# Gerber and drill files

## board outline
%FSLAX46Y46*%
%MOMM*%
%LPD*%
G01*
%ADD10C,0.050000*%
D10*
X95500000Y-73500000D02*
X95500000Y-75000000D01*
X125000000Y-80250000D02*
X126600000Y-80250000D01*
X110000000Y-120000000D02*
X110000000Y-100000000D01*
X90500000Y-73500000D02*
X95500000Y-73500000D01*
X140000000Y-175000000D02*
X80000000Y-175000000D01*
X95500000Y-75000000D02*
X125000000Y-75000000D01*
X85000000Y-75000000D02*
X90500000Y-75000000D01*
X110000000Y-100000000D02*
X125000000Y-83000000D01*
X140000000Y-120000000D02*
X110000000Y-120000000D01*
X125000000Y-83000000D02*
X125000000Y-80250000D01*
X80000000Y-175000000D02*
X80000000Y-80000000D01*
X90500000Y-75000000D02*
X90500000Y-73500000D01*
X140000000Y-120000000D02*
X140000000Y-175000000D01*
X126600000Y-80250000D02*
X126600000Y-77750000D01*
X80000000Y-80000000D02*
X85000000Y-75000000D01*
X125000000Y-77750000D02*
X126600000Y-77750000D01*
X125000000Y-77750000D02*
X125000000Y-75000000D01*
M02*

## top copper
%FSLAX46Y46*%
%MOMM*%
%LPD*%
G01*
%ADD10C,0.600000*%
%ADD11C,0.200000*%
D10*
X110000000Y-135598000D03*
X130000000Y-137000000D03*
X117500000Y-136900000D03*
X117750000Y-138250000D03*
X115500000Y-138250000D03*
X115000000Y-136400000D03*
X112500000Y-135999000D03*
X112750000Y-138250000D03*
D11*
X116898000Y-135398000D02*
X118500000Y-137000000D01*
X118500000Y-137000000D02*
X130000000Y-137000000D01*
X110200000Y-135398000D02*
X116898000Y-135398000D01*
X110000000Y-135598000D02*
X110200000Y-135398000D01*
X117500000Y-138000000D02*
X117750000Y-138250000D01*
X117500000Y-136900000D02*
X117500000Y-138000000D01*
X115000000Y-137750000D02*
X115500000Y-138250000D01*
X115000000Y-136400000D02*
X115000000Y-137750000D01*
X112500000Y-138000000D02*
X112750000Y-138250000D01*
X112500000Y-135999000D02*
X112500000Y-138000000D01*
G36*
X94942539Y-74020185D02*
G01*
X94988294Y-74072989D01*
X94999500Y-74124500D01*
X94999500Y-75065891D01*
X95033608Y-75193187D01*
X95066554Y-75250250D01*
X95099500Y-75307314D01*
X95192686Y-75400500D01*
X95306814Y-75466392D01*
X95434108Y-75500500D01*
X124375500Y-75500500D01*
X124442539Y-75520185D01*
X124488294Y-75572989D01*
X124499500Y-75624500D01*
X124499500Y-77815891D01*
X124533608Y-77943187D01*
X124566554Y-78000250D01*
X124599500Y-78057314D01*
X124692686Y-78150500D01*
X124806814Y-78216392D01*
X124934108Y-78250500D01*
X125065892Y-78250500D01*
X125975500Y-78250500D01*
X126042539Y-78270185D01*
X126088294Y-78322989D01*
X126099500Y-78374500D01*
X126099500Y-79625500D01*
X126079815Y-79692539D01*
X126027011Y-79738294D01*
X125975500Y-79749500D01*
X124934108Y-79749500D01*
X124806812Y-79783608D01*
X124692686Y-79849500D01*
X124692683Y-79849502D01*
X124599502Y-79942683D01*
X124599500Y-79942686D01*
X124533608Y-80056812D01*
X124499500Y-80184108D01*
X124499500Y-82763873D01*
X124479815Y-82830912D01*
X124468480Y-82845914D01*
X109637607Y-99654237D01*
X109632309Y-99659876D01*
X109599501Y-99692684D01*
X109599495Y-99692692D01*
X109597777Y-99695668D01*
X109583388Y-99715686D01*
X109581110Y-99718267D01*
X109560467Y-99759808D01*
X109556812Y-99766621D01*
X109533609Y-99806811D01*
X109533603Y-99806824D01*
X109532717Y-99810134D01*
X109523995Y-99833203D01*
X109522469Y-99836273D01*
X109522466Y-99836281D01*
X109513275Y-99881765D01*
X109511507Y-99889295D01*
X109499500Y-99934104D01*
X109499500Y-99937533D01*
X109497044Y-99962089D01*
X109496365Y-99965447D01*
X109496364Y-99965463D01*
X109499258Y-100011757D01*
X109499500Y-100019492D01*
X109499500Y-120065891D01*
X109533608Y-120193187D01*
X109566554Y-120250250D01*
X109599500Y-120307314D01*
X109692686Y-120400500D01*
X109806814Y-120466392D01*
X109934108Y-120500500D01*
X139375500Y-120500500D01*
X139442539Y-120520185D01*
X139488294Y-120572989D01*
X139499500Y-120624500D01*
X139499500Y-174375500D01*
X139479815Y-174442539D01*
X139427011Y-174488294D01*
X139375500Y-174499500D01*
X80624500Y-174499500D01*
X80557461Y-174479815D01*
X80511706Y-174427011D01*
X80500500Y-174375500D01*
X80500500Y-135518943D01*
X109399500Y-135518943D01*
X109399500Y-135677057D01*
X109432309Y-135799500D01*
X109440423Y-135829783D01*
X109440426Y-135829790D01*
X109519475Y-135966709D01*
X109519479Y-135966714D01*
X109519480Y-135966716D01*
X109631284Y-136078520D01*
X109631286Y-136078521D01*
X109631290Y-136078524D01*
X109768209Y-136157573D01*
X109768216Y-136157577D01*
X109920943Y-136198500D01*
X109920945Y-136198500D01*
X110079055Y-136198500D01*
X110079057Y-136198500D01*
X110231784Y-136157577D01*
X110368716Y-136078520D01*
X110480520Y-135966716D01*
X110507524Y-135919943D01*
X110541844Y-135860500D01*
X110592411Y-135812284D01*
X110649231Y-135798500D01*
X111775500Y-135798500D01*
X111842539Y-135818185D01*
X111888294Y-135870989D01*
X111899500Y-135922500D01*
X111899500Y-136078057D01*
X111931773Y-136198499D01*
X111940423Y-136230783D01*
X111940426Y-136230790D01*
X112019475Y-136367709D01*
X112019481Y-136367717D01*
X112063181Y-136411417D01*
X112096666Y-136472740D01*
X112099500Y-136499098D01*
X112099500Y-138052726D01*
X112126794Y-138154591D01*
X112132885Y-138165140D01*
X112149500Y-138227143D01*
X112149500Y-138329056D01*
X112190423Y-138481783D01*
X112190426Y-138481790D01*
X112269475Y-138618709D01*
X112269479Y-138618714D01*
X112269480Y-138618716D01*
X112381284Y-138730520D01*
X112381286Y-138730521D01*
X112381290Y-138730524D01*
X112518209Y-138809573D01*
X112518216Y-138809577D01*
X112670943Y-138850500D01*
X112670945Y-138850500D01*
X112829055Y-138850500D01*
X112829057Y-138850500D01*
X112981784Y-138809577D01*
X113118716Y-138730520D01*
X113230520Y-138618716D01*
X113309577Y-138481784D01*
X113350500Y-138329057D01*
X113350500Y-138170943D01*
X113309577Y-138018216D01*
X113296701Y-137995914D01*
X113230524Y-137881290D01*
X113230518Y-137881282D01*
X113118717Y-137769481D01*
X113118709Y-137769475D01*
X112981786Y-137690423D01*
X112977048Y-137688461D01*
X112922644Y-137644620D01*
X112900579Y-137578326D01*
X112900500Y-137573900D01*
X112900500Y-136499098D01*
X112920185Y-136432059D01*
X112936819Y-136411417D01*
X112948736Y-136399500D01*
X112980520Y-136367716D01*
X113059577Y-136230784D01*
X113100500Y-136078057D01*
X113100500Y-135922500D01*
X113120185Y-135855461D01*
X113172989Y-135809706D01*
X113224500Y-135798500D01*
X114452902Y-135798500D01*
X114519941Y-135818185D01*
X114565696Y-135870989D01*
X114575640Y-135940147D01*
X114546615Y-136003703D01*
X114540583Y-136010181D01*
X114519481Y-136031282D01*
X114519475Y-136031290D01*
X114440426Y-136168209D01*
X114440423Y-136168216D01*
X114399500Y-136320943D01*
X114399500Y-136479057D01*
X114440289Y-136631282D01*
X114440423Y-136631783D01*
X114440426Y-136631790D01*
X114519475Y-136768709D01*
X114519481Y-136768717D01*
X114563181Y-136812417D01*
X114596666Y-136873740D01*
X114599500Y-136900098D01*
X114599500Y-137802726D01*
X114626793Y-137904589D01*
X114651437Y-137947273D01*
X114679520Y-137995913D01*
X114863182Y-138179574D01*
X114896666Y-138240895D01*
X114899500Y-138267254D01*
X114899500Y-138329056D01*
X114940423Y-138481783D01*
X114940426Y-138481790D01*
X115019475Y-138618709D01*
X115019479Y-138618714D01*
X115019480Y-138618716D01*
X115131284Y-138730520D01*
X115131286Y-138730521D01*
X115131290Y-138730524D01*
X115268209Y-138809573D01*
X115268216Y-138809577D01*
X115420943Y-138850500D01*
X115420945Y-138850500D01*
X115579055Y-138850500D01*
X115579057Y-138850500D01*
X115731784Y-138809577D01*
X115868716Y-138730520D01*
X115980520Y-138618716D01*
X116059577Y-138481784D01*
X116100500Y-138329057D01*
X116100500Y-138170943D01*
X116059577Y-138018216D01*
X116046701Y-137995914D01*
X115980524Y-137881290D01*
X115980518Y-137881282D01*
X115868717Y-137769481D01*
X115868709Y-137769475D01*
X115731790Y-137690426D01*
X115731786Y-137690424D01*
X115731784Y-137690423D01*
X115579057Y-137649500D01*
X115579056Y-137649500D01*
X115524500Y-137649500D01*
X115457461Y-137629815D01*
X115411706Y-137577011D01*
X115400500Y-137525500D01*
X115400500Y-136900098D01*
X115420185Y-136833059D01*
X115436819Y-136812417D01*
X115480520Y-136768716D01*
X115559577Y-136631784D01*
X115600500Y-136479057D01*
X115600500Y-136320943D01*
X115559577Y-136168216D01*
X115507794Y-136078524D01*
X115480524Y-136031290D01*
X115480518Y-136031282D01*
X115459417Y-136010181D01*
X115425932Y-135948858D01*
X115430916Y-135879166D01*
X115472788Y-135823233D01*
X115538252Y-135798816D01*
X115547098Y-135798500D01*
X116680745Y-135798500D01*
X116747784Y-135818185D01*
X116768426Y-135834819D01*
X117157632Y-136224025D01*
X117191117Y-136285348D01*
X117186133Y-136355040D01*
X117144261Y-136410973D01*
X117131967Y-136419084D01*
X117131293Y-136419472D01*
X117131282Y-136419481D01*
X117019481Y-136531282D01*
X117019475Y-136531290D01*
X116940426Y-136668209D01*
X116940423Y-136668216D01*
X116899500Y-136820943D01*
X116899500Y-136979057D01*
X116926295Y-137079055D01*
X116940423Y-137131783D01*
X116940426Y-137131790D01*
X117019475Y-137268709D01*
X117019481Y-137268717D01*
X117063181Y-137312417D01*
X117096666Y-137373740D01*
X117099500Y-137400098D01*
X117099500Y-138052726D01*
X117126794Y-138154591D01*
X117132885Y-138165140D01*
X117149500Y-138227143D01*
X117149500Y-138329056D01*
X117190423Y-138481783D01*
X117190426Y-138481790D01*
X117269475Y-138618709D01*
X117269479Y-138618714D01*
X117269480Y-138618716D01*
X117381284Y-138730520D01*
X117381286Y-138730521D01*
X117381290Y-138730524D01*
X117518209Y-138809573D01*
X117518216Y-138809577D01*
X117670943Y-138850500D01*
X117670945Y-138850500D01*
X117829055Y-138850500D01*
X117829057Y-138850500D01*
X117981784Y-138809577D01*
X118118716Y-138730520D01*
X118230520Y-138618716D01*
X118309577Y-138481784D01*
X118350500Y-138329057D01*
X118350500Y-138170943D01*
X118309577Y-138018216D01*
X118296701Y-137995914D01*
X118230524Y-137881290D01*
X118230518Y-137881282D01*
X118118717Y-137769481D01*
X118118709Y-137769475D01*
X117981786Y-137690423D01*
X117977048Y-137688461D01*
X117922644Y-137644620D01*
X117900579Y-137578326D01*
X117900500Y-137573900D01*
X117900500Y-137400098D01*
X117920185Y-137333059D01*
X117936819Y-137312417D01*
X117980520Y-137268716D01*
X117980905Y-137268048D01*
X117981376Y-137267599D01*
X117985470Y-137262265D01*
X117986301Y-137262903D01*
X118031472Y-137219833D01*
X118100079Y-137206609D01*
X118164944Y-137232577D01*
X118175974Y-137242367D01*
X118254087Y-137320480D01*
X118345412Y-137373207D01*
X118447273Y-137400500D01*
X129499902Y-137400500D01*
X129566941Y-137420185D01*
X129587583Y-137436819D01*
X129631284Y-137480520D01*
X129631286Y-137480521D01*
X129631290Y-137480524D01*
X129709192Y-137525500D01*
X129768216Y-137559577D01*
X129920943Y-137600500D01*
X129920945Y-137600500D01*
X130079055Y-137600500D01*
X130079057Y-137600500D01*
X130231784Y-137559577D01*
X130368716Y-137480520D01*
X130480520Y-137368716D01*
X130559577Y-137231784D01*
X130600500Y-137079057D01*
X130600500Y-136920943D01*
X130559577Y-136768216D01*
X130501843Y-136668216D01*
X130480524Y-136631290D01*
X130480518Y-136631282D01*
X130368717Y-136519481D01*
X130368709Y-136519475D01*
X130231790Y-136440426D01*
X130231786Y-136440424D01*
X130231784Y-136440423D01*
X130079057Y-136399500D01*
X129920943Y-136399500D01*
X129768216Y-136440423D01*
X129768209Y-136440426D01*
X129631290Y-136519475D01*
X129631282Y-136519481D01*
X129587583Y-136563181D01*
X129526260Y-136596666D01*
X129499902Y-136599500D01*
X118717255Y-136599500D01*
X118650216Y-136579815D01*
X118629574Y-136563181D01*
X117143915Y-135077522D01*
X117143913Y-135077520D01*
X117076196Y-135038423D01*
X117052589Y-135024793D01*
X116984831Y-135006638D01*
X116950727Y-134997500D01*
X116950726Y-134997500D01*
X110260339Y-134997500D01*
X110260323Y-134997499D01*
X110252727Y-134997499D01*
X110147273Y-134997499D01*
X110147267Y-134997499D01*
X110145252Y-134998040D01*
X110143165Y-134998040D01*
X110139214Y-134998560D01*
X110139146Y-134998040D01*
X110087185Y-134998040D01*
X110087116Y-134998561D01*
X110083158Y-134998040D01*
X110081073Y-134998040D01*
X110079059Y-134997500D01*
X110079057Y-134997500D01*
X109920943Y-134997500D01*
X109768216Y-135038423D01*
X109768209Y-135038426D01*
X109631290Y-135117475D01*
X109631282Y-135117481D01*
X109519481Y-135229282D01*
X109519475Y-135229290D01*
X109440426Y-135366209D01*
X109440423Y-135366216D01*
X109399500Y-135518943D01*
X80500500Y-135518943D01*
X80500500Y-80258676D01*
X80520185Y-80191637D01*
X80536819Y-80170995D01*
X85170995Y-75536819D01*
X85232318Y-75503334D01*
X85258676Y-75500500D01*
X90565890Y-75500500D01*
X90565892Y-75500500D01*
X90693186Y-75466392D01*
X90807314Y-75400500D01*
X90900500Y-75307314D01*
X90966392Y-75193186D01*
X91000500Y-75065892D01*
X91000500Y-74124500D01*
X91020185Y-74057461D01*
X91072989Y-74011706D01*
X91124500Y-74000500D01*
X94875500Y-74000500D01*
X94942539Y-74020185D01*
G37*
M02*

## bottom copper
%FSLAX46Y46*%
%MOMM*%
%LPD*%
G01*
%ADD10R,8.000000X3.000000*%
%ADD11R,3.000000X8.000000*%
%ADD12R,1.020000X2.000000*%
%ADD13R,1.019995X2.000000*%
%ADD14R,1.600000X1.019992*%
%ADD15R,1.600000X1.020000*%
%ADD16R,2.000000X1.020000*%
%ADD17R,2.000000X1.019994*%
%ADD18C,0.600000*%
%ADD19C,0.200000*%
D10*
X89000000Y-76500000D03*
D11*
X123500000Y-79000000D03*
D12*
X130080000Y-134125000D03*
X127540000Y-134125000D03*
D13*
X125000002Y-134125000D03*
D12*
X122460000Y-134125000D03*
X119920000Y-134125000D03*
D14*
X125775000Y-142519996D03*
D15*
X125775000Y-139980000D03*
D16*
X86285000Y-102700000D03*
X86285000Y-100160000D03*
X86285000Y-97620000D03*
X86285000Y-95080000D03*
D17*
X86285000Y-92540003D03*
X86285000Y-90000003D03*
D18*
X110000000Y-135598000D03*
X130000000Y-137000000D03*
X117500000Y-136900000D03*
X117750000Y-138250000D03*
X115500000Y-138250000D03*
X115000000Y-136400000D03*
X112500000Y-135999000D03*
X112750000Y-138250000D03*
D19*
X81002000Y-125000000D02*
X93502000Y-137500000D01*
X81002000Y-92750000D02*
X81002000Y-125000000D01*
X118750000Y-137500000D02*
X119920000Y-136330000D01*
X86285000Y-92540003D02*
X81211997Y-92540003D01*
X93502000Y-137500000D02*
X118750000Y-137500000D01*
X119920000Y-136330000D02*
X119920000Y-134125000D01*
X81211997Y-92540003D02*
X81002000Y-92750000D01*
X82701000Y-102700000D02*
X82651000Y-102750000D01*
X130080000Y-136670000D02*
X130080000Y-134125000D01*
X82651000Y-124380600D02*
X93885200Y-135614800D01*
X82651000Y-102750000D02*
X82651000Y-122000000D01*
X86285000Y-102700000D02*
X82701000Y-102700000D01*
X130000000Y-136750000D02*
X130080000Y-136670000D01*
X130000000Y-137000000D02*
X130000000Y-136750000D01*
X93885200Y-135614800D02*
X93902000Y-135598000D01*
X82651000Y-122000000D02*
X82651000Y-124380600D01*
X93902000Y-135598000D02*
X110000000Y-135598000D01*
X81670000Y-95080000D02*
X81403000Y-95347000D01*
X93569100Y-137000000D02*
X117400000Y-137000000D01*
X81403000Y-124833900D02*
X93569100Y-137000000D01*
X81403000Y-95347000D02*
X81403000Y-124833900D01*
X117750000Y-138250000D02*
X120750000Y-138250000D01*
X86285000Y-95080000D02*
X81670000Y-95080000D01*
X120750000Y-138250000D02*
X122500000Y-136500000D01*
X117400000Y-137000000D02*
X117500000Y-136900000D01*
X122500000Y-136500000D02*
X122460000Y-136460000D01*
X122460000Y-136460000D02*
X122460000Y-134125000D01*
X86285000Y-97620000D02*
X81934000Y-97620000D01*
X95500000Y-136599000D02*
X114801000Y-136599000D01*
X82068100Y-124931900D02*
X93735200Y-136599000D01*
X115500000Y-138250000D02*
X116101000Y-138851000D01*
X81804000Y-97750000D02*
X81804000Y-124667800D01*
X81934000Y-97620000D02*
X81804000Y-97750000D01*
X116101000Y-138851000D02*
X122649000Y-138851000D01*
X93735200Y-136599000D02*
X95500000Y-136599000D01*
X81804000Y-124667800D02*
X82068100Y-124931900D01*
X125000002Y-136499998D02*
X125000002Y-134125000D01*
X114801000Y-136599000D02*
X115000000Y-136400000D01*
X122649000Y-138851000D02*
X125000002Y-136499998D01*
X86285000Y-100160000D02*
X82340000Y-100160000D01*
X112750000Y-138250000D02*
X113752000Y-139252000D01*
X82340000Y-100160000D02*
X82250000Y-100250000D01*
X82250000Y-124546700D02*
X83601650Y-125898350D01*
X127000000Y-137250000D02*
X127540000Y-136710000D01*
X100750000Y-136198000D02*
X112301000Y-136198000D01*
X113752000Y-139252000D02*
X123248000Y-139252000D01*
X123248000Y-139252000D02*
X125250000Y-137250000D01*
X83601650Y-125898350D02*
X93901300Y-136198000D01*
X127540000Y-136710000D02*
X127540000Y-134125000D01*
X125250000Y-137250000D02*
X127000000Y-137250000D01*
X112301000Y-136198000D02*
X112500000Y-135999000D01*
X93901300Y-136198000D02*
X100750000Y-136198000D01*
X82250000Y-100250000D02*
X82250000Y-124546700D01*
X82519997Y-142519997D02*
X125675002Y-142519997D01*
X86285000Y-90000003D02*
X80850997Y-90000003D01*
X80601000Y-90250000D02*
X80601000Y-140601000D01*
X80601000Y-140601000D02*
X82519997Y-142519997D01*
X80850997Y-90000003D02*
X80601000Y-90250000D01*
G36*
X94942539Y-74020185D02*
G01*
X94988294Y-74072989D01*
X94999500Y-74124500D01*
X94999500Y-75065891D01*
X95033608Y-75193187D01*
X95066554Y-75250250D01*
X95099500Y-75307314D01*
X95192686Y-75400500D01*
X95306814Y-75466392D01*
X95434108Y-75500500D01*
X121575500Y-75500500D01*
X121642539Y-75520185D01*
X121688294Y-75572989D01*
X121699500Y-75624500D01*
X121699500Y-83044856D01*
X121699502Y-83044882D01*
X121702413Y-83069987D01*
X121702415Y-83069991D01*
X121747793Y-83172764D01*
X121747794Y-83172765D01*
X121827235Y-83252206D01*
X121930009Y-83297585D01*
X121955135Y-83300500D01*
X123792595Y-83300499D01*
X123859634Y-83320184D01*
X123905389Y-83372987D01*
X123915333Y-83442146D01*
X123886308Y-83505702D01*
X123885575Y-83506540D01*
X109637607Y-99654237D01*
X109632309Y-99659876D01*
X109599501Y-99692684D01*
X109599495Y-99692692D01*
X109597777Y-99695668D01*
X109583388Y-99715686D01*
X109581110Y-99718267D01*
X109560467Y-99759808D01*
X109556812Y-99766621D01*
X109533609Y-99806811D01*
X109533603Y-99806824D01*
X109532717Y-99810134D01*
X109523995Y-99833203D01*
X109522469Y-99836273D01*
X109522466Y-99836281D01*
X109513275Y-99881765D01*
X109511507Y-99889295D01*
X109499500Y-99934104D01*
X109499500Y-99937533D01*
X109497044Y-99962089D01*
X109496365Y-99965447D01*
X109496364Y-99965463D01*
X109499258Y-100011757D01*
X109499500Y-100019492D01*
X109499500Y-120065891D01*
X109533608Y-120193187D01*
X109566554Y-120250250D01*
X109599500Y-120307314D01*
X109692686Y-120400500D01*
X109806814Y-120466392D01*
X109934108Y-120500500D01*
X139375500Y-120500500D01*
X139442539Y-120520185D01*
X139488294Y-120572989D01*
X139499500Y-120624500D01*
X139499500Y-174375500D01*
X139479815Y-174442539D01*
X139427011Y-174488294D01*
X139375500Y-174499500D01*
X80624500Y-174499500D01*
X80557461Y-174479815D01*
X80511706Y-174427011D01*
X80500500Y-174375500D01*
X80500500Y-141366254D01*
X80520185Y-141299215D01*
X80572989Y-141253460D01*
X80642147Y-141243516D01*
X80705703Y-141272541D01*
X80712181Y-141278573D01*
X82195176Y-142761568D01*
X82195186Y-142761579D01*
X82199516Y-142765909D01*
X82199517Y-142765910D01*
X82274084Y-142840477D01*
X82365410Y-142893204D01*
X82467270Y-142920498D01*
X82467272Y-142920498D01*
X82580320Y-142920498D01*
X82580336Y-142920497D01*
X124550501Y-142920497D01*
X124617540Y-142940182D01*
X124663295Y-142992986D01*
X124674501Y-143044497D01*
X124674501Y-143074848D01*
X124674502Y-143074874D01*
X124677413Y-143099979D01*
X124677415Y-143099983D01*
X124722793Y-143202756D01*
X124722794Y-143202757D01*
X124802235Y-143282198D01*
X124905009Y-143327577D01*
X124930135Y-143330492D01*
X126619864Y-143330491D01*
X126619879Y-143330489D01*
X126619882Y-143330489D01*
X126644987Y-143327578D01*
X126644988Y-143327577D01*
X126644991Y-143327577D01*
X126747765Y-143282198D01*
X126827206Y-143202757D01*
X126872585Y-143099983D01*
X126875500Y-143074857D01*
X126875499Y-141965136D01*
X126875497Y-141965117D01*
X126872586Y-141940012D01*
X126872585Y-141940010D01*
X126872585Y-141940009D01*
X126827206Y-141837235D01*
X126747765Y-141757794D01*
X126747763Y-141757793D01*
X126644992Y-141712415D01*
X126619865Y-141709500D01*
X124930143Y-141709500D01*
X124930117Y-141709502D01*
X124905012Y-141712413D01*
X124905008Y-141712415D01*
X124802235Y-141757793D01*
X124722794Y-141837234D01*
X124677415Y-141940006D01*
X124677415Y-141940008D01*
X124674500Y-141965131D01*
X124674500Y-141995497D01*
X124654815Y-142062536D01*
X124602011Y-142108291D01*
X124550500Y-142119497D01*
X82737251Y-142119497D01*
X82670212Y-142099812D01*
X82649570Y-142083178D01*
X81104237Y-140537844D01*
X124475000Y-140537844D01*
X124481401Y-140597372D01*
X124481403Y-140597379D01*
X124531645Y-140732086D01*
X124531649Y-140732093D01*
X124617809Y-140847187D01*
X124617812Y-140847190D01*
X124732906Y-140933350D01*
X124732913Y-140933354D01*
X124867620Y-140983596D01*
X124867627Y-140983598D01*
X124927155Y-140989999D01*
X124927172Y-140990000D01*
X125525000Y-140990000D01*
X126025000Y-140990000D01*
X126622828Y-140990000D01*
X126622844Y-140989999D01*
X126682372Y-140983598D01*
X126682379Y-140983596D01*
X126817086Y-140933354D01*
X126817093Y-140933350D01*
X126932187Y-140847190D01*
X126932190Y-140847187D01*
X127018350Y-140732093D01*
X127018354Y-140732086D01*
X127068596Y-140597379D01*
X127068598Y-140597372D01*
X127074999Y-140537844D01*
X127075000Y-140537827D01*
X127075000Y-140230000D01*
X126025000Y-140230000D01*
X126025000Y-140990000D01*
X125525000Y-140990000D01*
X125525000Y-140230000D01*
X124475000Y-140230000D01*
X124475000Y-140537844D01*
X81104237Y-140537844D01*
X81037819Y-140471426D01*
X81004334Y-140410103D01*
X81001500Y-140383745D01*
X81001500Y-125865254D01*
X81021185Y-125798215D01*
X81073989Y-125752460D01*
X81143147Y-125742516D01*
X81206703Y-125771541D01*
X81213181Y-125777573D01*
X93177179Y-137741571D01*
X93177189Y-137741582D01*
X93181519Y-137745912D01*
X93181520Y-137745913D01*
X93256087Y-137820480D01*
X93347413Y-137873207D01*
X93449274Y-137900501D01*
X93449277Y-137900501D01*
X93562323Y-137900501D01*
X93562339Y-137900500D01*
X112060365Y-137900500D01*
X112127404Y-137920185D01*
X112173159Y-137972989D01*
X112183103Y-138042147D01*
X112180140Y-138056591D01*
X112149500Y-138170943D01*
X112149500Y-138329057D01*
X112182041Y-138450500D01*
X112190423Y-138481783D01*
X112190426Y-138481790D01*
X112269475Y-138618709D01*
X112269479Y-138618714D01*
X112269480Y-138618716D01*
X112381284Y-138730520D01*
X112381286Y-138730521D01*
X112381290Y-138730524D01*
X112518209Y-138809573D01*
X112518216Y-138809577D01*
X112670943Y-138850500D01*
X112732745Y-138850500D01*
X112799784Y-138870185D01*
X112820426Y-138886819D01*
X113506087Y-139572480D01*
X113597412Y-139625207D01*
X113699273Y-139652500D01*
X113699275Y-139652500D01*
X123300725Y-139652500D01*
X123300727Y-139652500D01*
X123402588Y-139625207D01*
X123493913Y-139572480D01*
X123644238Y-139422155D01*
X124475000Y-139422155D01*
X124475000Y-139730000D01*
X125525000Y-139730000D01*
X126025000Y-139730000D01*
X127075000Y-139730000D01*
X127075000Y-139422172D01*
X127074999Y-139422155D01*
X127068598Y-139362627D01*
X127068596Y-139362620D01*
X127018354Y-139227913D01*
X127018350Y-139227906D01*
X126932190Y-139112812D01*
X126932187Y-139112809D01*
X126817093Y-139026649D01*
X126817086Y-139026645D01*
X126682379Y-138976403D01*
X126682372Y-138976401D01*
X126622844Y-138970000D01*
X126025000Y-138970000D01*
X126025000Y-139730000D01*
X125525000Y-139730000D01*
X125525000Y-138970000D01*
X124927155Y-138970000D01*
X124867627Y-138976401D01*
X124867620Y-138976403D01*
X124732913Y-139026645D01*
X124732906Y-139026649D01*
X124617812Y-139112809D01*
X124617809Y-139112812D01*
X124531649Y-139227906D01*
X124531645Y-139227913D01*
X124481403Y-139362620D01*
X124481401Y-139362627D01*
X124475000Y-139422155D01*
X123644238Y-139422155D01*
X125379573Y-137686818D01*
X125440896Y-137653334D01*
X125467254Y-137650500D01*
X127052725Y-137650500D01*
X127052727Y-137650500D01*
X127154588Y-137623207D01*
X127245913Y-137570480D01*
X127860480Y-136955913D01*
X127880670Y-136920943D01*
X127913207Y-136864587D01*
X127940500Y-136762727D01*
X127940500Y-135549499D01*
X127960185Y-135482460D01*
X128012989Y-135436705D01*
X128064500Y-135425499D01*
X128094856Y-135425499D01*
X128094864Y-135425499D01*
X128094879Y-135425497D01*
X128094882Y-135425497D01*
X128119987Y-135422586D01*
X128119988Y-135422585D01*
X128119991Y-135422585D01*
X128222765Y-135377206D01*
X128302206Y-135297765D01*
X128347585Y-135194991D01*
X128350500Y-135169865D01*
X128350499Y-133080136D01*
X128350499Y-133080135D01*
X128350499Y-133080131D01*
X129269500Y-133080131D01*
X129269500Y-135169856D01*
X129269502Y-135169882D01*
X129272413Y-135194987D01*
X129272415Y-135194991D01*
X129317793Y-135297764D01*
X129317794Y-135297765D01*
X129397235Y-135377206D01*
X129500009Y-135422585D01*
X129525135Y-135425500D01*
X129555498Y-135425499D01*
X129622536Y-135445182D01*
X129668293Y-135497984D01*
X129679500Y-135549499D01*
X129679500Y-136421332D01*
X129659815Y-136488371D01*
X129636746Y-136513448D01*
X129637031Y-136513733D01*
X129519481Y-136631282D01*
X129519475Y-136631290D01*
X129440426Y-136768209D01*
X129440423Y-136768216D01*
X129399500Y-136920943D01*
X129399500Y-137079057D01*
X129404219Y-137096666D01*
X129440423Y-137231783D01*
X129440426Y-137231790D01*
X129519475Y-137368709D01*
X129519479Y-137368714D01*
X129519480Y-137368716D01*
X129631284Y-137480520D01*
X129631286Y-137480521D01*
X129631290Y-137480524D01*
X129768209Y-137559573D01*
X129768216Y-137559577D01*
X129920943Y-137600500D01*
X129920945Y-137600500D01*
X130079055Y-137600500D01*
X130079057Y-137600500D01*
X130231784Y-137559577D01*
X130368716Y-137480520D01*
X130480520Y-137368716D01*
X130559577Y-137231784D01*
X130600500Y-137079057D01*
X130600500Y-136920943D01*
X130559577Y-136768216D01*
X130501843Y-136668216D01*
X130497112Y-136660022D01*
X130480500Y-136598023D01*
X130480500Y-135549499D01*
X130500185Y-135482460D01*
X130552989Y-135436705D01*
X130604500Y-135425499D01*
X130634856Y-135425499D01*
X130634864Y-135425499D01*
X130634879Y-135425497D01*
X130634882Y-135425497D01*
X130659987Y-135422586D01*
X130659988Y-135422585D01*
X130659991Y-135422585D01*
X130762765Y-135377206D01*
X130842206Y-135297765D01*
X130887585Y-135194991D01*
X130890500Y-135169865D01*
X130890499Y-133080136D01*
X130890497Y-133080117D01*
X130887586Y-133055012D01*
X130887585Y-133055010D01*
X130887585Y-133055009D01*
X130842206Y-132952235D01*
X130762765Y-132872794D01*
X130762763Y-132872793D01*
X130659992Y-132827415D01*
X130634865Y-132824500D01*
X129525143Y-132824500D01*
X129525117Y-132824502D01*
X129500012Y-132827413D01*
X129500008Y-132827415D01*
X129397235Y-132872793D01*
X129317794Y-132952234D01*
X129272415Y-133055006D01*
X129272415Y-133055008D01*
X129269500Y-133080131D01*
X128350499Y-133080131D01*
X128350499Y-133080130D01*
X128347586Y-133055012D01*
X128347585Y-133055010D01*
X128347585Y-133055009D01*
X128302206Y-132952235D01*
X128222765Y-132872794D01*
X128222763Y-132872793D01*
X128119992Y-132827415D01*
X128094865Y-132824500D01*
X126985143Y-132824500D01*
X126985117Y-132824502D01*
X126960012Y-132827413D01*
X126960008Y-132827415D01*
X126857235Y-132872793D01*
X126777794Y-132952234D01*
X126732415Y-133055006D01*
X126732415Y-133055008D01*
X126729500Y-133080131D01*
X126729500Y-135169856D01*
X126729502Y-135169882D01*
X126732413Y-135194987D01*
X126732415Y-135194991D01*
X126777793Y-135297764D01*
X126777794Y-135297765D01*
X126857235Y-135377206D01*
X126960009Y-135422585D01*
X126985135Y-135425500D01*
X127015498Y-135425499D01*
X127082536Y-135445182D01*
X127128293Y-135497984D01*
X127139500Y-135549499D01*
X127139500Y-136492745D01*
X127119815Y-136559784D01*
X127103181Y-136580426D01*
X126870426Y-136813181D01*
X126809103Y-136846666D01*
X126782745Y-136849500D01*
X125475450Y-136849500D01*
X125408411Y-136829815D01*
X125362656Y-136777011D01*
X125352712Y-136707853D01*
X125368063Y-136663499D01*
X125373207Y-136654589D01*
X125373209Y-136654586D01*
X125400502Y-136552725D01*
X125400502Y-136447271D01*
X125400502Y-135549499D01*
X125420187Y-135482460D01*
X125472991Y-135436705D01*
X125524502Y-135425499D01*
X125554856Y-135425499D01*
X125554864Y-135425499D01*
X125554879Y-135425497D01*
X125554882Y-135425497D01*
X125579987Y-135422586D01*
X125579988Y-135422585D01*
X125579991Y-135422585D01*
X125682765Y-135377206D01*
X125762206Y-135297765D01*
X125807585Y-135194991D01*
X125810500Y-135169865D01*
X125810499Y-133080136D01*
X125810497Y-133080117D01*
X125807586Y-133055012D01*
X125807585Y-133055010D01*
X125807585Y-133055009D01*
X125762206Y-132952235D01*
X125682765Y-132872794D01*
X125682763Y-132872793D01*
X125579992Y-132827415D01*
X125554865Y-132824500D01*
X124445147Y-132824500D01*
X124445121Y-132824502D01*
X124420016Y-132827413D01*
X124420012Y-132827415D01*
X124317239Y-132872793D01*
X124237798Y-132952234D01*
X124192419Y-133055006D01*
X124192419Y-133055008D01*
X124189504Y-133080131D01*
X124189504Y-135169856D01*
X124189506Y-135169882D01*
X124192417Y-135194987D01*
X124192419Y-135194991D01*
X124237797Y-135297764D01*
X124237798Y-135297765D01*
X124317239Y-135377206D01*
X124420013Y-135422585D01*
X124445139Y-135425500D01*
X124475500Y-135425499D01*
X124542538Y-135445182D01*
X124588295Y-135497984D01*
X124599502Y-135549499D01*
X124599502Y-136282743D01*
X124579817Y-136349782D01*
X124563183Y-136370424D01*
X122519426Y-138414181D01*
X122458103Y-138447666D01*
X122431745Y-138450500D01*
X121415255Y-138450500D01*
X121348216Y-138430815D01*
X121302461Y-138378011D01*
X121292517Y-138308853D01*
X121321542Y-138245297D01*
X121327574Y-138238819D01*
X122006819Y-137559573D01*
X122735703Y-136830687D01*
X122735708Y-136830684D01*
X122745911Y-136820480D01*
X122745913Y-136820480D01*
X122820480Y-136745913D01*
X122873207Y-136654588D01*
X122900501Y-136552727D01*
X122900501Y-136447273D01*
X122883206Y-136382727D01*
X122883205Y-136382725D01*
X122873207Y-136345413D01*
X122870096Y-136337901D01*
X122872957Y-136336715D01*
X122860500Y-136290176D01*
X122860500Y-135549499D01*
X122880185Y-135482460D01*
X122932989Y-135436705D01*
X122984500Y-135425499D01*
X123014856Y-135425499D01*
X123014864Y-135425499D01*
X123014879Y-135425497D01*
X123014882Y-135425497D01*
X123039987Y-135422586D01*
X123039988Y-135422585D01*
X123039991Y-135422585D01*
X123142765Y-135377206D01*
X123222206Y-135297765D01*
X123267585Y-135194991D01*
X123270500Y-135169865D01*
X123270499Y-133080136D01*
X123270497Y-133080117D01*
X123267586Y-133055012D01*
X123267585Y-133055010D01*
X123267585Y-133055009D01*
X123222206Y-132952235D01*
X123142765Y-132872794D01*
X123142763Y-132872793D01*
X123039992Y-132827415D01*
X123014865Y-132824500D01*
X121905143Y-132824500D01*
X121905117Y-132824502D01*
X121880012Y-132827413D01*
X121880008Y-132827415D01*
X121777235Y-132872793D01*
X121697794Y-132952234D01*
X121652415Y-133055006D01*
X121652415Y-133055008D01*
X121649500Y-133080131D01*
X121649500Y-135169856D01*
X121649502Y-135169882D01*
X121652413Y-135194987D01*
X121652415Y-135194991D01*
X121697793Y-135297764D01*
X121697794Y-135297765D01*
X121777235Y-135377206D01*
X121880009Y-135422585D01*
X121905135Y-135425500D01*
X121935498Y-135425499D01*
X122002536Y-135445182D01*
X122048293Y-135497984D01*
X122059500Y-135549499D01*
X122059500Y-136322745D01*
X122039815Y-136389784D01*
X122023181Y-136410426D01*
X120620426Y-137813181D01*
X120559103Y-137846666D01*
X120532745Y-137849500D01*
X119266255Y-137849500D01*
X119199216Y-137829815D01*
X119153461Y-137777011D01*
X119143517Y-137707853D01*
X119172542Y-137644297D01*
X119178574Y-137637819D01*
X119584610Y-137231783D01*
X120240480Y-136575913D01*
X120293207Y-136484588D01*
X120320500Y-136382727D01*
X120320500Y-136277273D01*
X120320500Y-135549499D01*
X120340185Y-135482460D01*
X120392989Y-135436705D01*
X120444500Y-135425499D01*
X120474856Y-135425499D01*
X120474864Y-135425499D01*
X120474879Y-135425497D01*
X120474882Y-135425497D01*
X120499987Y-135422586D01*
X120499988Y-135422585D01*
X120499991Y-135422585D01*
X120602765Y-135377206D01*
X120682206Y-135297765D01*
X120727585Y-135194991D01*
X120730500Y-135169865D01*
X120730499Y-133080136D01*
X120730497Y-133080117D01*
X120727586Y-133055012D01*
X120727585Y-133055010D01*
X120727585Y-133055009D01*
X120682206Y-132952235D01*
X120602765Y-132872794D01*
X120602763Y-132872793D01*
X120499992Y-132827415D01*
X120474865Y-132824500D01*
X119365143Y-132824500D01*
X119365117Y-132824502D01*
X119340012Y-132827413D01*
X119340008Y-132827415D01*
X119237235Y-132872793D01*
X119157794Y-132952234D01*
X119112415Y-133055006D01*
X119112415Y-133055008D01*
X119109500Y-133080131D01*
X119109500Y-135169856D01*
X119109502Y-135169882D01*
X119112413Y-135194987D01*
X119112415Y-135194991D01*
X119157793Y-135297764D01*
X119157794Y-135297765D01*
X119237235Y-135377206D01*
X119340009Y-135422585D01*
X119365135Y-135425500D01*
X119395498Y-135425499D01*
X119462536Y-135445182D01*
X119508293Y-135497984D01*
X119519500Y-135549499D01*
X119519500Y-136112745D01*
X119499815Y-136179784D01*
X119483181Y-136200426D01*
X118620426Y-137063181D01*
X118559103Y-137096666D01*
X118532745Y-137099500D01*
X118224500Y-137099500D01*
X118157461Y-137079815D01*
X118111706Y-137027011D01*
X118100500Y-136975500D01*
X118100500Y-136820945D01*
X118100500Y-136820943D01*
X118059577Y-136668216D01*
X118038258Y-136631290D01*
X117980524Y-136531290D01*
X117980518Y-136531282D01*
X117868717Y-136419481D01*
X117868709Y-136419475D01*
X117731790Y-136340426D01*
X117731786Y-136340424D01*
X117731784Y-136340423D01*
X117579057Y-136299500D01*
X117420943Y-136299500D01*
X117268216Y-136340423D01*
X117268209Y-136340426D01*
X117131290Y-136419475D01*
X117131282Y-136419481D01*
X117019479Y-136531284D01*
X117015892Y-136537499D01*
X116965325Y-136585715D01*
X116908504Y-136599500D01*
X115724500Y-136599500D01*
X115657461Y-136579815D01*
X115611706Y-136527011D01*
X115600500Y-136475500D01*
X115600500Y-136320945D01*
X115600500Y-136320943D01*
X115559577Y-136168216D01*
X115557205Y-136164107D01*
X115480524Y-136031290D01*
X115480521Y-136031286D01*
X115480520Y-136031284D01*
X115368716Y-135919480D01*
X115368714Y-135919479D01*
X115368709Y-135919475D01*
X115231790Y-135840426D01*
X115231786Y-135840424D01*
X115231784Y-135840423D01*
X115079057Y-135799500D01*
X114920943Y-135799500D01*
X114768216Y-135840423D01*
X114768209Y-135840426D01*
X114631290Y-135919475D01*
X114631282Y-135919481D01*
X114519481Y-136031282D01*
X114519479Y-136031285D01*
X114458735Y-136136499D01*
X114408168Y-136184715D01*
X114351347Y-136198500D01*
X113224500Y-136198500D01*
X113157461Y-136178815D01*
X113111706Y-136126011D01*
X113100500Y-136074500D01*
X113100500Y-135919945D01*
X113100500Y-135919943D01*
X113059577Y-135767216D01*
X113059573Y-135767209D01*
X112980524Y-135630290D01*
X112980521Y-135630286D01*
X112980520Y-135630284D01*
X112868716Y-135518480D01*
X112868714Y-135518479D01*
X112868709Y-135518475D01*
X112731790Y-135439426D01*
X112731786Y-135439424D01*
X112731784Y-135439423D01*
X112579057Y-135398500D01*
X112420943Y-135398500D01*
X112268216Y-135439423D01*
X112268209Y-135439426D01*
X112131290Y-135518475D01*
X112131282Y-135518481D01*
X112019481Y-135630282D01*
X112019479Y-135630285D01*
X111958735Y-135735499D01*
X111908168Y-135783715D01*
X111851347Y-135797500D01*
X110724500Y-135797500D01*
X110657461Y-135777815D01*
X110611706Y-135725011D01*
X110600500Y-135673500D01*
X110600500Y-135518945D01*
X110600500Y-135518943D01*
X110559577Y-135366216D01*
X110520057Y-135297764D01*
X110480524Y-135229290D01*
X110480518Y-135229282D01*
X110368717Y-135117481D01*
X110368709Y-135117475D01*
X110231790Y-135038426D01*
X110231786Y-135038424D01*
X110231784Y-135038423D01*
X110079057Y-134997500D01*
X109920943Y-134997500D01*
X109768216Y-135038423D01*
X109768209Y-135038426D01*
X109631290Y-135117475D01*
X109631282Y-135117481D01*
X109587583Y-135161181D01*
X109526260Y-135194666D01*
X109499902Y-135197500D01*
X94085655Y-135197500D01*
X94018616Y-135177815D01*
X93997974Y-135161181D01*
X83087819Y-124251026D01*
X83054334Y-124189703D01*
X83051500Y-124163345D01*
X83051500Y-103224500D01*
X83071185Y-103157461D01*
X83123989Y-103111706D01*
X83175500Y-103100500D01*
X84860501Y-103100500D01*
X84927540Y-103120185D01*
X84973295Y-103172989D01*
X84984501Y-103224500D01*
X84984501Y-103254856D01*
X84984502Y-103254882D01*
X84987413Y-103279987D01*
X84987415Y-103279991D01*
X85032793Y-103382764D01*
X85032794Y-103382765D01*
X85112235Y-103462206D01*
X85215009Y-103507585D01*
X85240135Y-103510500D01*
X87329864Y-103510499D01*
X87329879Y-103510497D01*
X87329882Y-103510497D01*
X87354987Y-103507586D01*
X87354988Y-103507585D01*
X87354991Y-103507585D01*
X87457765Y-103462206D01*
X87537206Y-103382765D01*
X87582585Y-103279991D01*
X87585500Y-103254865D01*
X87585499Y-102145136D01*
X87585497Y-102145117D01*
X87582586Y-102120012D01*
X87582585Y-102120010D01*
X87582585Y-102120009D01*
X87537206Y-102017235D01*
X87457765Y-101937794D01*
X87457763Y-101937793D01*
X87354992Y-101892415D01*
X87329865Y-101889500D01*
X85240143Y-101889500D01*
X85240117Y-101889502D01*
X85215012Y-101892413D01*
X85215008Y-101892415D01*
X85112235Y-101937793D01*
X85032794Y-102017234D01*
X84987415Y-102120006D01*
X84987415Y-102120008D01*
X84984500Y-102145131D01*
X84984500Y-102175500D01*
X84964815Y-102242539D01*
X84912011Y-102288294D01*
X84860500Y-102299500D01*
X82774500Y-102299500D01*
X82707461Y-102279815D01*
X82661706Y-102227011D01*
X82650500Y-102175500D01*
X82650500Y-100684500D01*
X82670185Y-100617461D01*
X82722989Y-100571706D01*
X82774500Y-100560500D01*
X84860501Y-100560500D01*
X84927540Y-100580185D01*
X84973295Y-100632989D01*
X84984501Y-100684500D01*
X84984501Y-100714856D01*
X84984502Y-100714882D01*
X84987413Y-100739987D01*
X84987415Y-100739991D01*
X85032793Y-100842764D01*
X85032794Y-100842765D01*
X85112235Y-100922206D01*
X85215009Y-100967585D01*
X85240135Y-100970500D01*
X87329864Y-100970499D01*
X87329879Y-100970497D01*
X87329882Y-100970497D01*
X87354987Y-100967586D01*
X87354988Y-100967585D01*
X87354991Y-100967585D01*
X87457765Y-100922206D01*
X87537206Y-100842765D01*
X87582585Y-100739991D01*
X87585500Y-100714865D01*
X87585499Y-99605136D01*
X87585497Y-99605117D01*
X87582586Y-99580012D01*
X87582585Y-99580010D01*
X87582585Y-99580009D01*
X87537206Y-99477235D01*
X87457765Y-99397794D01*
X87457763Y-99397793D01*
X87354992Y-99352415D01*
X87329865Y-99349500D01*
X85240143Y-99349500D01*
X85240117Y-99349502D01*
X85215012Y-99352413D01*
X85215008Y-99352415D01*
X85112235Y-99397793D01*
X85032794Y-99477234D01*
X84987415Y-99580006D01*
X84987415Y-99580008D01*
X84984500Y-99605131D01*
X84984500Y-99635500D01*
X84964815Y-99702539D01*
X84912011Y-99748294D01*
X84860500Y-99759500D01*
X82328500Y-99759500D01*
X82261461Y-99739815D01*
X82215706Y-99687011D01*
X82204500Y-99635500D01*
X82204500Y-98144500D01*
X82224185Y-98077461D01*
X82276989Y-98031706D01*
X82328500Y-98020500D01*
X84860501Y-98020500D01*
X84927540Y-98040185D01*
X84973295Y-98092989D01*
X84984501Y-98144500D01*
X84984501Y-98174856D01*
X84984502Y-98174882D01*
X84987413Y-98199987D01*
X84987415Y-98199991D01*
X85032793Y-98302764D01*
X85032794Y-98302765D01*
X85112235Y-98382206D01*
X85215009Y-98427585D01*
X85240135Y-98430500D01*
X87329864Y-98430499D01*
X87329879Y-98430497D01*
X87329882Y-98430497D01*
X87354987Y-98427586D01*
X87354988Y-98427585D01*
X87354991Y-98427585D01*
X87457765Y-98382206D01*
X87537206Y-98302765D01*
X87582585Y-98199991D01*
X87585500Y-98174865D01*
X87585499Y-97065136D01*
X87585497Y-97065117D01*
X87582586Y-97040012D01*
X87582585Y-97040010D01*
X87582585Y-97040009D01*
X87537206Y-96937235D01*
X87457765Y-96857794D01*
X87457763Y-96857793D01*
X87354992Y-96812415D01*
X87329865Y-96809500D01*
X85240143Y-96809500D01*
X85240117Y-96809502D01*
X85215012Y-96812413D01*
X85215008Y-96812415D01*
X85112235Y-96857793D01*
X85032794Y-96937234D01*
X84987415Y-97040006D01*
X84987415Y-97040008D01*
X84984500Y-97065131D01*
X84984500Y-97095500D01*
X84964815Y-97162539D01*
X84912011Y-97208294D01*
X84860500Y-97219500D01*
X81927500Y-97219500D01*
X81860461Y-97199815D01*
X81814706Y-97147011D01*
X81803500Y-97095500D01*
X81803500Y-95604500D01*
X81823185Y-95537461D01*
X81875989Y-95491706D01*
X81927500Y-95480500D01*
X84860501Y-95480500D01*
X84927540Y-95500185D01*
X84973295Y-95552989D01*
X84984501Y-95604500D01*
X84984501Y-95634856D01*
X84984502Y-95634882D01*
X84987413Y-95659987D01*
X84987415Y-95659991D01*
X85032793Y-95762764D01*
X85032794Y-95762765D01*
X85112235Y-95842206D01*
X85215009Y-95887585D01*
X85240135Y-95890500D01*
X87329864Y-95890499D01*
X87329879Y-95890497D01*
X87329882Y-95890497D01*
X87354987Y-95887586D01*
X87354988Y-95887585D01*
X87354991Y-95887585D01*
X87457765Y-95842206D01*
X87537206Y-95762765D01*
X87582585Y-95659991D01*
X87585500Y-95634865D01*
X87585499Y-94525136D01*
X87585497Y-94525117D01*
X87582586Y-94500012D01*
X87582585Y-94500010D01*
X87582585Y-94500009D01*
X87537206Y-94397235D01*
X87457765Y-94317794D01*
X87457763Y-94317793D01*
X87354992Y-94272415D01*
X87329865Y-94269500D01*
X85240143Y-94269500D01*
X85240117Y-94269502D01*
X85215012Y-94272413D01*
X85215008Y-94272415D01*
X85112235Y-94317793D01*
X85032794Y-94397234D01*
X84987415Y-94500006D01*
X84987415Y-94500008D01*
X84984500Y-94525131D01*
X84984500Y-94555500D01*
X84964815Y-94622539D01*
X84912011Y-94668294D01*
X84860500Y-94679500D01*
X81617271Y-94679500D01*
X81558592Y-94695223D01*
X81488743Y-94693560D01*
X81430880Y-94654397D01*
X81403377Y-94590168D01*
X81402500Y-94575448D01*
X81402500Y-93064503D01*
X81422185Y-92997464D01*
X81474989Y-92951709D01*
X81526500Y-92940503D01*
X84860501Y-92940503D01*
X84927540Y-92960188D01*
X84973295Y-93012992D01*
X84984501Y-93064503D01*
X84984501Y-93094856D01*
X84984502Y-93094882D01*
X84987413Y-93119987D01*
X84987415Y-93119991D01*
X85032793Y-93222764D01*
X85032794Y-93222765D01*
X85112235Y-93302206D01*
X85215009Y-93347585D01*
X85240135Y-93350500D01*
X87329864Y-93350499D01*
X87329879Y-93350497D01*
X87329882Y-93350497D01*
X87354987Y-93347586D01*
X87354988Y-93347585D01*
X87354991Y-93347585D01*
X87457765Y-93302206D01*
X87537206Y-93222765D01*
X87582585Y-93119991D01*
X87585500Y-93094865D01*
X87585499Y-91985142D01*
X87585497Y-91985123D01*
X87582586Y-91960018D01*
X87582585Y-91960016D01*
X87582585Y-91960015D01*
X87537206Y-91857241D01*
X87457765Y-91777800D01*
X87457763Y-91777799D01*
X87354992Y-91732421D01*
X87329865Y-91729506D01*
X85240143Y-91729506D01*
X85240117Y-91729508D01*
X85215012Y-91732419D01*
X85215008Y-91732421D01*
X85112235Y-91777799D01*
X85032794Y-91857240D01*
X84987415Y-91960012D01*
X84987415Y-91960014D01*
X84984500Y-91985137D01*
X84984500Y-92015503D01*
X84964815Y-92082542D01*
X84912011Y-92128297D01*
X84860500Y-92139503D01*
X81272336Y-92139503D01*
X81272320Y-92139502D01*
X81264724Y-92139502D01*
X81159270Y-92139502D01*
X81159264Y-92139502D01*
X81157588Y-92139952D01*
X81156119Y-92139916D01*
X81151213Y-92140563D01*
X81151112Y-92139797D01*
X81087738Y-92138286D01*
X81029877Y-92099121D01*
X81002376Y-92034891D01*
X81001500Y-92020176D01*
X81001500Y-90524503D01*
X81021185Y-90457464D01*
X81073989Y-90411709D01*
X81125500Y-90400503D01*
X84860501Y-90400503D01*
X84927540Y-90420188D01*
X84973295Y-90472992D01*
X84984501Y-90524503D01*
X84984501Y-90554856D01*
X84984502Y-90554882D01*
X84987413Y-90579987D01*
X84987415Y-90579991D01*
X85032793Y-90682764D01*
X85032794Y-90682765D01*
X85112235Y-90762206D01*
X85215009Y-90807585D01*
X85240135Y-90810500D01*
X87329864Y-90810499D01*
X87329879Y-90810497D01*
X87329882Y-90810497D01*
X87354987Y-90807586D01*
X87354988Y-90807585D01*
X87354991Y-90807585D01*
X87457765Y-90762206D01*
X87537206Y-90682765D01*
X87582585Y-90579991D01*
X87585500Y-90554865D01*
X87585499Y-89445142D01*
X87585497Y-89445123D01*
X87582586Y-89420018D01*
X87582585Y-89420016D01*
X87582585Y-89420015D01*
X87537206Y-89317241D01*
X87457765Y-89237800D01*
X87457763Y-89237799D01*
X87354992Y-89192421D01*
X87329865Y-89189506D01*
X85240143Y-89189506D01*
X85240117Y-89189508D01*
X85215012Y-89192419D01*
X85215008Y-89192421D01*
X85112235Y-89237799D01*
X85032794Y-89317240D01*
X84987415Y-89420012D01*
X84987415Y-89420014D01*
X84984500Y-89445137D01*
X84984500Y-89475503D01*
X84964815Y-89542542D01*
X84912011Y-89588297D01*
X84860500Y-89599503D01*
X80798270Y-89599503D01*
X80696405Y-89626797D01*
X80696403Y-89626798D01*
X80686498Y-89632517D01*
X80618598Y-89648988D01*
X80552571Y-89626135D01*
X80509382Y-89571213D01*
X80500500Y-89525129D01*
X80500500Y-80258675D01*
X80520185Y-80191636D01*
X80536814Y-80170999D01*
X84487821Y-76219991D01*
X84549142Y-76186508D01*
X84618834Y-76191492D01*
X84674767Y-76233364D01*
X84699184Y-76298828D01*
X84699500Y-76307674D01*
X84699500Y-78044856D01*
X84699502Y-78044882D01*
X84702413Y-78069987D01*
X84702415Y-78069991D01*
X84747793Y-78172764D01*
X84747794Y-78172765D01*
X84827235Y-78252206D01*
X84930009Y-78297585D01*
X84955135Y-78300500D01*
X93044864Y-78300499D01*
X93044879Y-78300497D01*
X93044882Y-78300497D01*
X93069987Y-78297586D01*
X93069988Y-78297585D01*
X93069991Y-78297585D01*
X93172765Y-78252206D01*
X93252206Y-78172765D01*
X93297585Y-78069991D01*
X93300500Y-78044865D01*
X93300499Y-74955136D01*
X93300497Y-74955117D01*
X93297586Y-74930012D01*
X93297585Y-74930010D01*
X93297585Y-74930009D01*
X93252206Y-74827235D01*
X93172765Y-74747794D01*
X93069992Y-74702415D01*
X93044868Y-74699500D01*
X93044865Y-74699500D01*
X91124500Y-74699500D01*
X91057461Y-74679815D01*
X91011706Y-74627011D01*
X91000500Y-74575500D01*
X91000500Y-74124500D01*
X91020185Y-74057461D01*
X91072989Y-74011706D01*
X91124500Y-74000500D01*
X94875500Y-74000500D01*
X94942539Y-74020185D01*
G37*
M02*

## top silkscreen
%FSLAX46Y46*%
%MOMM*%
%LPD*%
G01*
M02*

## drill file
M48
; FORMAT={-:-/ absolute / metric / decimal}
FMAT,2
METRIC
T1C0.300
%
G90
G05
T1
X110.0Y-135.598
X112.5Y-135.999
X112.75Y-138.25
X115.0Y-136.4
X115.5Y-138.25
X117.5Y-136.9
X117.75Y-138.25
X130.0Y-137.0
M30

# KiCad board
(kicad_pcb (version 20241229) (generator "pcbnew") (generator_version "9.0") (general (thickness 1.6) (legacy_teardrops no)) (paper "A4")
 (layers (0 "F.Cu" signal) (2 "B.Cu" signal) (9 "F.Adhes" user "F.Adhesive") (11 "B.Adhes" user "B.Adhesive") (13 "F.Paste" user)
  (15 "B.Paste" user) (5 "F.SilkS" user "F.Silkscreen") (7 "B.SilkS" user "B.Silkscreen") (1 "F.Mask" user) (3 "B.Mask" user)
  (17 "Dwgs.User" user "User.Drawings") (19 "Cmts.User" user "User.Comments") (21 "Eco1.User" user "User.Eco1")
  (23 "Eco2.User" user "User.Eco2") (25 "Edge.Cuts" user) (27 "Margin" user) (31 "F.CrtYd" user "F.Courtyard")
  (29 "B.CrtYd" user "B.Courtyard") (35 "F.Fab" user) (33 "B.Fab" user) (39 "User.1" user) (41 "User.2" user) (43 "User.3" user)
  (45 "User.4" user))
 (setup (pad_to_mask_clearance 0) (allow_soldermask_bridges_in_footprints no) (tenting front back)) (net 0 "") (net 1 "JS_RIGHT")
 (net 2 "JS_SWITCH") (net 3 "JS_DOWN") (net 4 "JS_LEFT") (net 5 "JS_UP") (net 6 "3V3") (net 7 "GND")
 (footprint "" (layer "F.Cu") (at 89 76.5 90)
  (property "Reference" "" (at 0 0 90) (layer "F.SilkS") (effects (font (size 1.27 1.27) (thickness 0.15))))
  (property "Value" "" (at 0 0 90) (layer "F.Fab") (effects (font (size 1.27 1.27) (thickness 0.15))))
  (pad "" smd rect (at 0 0 270) (size 3 8) (layers "B.Cu" "B.Mask" "B.Paste")))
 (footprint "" (layer "F.Cu") (at 123.6 79 90)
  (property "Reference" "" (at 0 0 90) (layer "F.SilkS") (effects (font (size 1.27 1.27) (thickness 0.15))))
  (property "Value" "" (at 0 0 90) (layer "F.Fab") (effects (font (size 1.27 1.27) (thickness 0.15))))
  (pad "" smd rect (at 0 -0.1 180) (size 3 8) (layers "B.Cu" "B.Mask" "B.Paste")))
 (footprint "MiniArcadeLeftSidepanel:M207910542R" (layer "B.Cu") (at 125 128.825 180)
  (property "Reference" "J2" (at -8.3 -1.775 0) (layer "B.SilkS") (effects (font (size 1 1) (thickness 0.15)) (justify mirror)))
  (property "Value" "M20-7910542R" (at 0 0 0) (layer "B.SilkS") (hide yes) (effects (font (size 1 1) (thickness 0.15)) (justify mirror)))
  (pad "1" smd rect (at -5.08 -5.3 180) (size 1.02 2) (layers "B.Cu" "B.Mask" "B.Paste") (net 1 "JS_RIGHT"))
  (pad "2" smd rect (at -2.54 -5.3 180) (size 1.02 2) (layers "B.Cu" "B.Mask" "B.Paste") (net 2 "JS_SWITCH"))
  (pad "3" smd rect (at -0.000002 -5.3 180) (size 1.019995 2) (layers "B.Cu" "B.Mask" "B.Paste") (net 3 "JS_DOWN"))
  (pad "4" smd rect (at 2.54 -5.3 180) (size 1.02 2) (layers "B.Cu" "B.Mask" "B.Paste") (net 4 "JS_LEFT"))
  (pad "5" smd rect (at 5.08 -5.3 180) (size 1.02 2) (layers "B.Cu" "B.Mask" "B.Paste") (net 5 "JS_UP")))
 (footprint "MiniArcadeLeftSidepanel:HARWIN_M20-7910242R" (layer "B.Cu") (at 133.175 141.25 -90)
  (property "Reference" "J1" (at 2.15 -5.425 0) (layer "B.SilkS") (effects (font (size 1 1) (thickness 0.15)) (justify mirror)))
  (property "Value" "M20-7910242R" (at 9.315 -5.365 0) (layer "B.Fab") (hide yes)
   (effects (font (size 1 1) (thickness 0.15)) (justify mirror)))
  (pad "1" smd rect (at 1.269996 7.4 270) (size 1.019992 1.6) (layers "B.Cu" "B.Mask" "B.Paste") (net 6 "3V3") (solder_mask_margin 0.102))
  (pad "2" smd rect (at -1.27 7.4 270) (size 1.02 1.6) (layers "B.Cu" "B.Mask" "B.Paste") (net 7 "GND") (solder_mask_margin 0.102)))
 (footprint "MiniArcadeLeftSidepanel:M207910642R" (layer "B.Cu") (at 91.585 96.35 90)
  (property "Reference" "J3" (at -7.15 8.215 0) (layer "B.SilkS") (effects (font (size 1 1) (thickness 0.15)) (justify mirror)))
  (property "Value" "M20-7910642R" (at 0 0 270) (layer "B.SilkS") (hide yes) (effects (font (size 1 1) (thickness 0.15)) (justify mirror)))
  (pad "1" smd rect (at -6.35 -5.3 90) (size 1.02 2) (layers "B.Cu" "B.Mask" "B.Paste") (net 1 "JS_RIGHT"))
  (pad "2" smd rect (at -3.81 -5.3 90) (size 1.02 2) (layers "B.Cu" "B.Mask" "B.Paste") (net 2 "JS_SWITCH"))
  (pad "3" smd rect (at -1.27 -5.3 90) (size 1.02 2) (layers "B.Cu" "B.Mask" "B.Paste") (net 3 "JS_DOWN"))
  (pad "4" smd rect (at 1.27 -5.3 90) (size 1.02 2) (layers "B.Cu" "B.Mask" "B.Paste") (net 4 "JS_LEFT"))
  (pad "5" smd rect (at 3.809997 -5.3 90) (size 1.019994 2) (layers "B.Cu" "B.Mask" "B.Paste") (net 5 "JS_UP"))
  (pad "6" smd rect (at 6.349997 -5.3 90) (size 1.019994 2) (layers "B.Cu" "B.Mask" "B.Paste") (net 6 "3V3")))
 (gr_line (start 95.5 73.5) (end 95.5 75) (stroke (width 0.05) (type default)) (layer "Edge.Cuts"))
 (gr_line (start 125 80.25) (end 126.6 80.25) (stroke (width 0.05) (type solid)) (layer "Edge.Cuts"))
 (gr_line (start 110 120) (end 110 100) (stroke (width 0.05) (type solid)) (layer "Edge.Cuts"))
 (gr_line (start 90.5 73.5) (end 95.5 73.5) (stroke (width 0.05) (type default)) (layer "Edge.Cuts"))
 (gr_line (start 140 175) (end 80 175) (stroke (width 0.05) (type solid)) (layer "Edge.Cuts"))
 (gr_line (start 95.5 75) (end 125 75) (stroke (width 0.05) (type default)) (layer "Edge.Cuts"))
 (gr_line (start 85 75) (end 90.5 75) (stroke (width 0.05) (type default)) (layer "Edge.Cuts"))
 (gr_line (start 110 100) (end 125 83) (stroke (width 0.05) (type default)) (layer "Edge.Cuts"))
 (gr_line (start 140 120) (end 110 120) (stroke (width 0.05) (type solid)) (layer "Edge.Cuts"))
 (gr_line (start 125 83) (end 125 80.25) (stroke (width 0.05) (type default)) (layer "Edge.Cuts"))
 (gr_line (start 80 175) (end 80 80) (stroke (width 0.05) (type solid)) (layer "Edge.Cuts"))
 (gr_line (start 90.5 75) (end 90.5 73.5) (stroke (width 0.05) (type default)) (layer "Edge.Cuts"))
 (gr_line (start 140 120) (end 140 175) (stroke (width 0.05) (type solid)) (layer "Edge.Cuts"))
 (gr_line (start 126.6 80.25) (end 126.6 77.75) (stroke (width 0.05) (type solid)) (layer "Edge.Cuts"))
 (gr_line (start 80 80) (end 85 75) (stroke (width 0.05) (type default)) (layer "Edge.Cuts"))
 (gr_line (start 125 77.75) (end 126.6 77.75) (stroke (width 0.05) (type solid)) (layer "Edge.Cuts"))
 (gr_line (start 125 77.75) (end 125 75) (stroke (width 0.05) (type default)) (layer "Edge.Cuts"))
 (segment (start 81.002 125) (end 93.502 137.5) (width 0.2) (layer "B.Cu") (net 5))
 (segment (start 81.002 92.75) (end 81.002 125) (width 0.2) (layer "B.Cu") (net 5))
 (segment (start 118.75 137.5) (end 119.92 136.33) (width 0.2) (layer "B.Cu") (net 5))
 (segment (start 86.285 92.540003) (end 81.211997 92.540003) (width 0.2) (layer "B.Cu") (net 5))
 (segment (start 93.502 137.5) (end 118.75 137.5) (width 0.2) (layer "B.Cu") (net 5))
 (segment (start 119.92 136.33) (end 119.92 134.125) (width 0.2) (layer "B.Cu") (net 5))
 (segment (start 81.211997 92.540003) (end 81.002 92.75) (width 0.2) (layer "B.Cu") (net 5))
 (segment (start 116.898 135.398) (end 118.5 137) (width 0.2) (layer "F.Cu") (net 1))
 (segment (start 118.5 137) (end 130 137) (width 0.2) (layer "F.Cu") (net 1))
 (segment (start 110.2 135.398) (end 116.898 135.398) (width 0.2) (layer "F.Cu") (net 1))
 (segment (start 110 135.598) (end 110.2 135.398) (width 0.2) (layer "F.Cu") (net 1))
 (via (at 110 135.598) (size 0.6) (drill 0.3) (layers "F.Cu" "B.Cu") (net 1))
 (via (at 130 137) (size 0.6) (drill 0.3) (layers "F.Cu" "B.Cu") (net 1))
 (segment (start 82.701 102.7) (end 82.651 102.75) (width 0.2) (layer "B.Cu") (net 1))
 (segment (start 130.08 136.67) (end 130.08 134.125) (width 0.2) (layer "B.Cu") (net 1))
 (segment (start 82.651 124.3806) (end 93.8852 135.6148) (width 0.2) (layer "B.Cu") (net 1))
 (segment (start 82.651 102.75) (end 82.651 122) (width 0.2) (layer "B.Cu") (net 1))
 (segment (start 86.285 102.7) (end 82.701 102.7) (width 0.2) (layer "B.Cu") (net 1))
 (segment (start 130 136.75) (end 130.08 136.67) (width 0.2) (layer "B.Cu") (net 1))
 (segment (start 130 137) (end 130 136.75) (width 0.2) (layer "B.Cu") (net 1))
 (segment (start 93.8852 135.6148) (end 93.902 135.598) (width 0.2) (layer "B.Cu") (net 1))
 (segment (start 82.651 122) (end 82.651 124.3806) (width 0.2) (layer "B.Cu") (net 1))
 (segment (start 93.902 135.598) (end 110 135.598) (width 0.2) (layer "B.Cu") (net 1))
 (segment (start 117.5 138) (end 117.75 138.25) (width 0.2) (layer "F.Cu") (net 4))
 (segment (start 117.5 136.9) (end 117.5 138) (width 0.2) (layer "F.Cu") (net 4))
 (via (at 117.5 136.9) (size 0.6) (drill 0.3) (layers "F.Cu" "B.Cu") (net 4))
 (via (at 117.75 138.25) (size 0.6) (drill 0.3) (layers "F.Cu" "B.Cu") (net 4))
 (segment (start 81.67 95.08) (end 81.403 95.347) (width 0.2) (layer "B.Cu") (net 4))
 (segment (start 93.5691 137) (end 117.4 137) (width 0.2) (layer "B.Cu") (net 4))
 (segment (start 81.403 124.8339) (end 93.5691 137) (width 0.2) (layer "B.Cu") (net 4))
 (segment (start 81.403 95.347) (end 81.403 124.8339) (width 0.2) (layer "B.Cu") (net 4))
 (segment (start 117.75 138.25) (end 120.75 138.25) (width 0.2) (layer "B.Cu") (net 4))
 (segment (start 86.285 95.08) (end 81.67 95.08) (width 0.2) (layer "B.Cu") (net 4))
 (segment (start 120.75 138.25) (end 122.5 136.5) (width 0.2) (layer "B.Cu") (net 4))
 (segment (start 117.4 137) (end 117.5 136.9) (width 0.2) (layer "B.Cu") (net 4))
 (segment (start 122.5 136.5) (end 122.46 136.46) (width 0.2) (layer "B.Cu") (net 4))
 (segment (start 122.46 136.46) (end 122.46 134.125) (width 0.2) (layer "B.Cu") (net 4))
 (segment (start 115 137.75) (end 115.5 138.25) (width 0.2) (layer "F.Cu") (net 3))
 (segment (start 115 136.4) (end 115 137.75) (width 0.2) (layer "F.Cu") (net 3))
 (via (at 115.5 138.25) (size 0.6) (drill 0.3) (layers "F.Cu" "B.Cu") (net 3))
 (via (at 115 136.4) (size 0.6) (drill 0.3) (layers "F.Cu" "B.Cu") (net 3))
 (segment (start 86.285 97.62) (end 81.934 97.62) (width 0.2) (layer "B.Cu") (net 3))
 (segment (start 95.5 136.599) (end 114.801 136.599) (width 0.2) (layer "B.Cu") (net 3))
 (segment (start 82.0681 124.9319) (end 93.7352 136.599) (width 0.2) (layer "B.Cu") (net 3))
 (segment (start 115.5 138.25) (end 116.101 138.851) (width 0.2) (layer "B.Cu") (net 3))
 (segment (start 81.804 97.75) (end 81.804 124.6678) (width 0.2) (layer "B.Cu") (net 3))
 (segment (start 81.934 97.62) (end 81.804 97.75) (width 0.2) (layer "B.Cu") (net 3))
 (segment (start 116.101 138.851) (end 122.649 138.851) (width 0.2) (layer "B.Cu") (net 3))
 (segment (start 93.7352 136.599) (end 95.5 136.599) (width 0.2) (layer "B.Cu") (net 3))
 (segment (start 81.804 124.6678) (end 82.0681 124.9319) (width 0.2) (layer "B.Cu") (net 3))
 (segment (start 125.000002 136.499998) (end 125.000002 134.125) (width 0.2) (layer "B.Cu") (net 3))
 (segment (start 114.801 136.599) (end 115 136.4) (width 0.2) (layer "B.Cu") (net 3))
 (segment (start 122.649 138.851) (end 125.000002 136.499998) (width 0.2) (layer "B.Cu") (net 3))
 (segment (start 112.5 138) (end 112.75 138.25) (width 0.2) (layer "F.Cu") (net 2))
 (segment (start 112.5 135.999) (end 112.5 138) (width 0.2) (layer "F.Cu") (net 2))
 (via (at 112.5 135.999) (size 0.6) (drill 0.3) (layers "F.Cu" "B.Cu") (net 2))
 (via (at 112.75 138.25) (size 0.6) (drill 0.3) (layers "F.Cu" "B.Cu") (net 2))
 (segment (start 86.285 100.16) (end 82.34 100.16) (width 0.2) (layer "B.Cu") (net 2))
 (segment (start 112.75 138.25) (end 113.752 139.252) (width 0.2) (layer "B.Cu") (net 2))
 (segment (start 82.34 100.16) (end 82.25 100.25) (width 0.2) (layer "B.Cu") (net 2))
 (segment (start 82.25 124.5467) (end 83.60165 125.89835) (width 0.2) (layer "B.Cu") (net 2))
 (segment (start 127 137.25) (end 127.54 136.71) (width 0.2) (layer "B.Cu") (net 2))
 (segment (start 100.75 136.198) (end 112.301 136.198) (width 0.2) (layer "B.Cu") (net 2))
 (segment (start 113.752 139.252) (end 123.248 139.252) (width 0.2) (layer "B.Cu") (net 2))
 (segment (start 123.248 139.252) (end 125.25 137.25) (width 0.2) (layer "B.Cu") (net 2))
 (segment (start 83.60165 125.89835) (end 93.9013 136.198) (width 0.2) (layer "B.Cu") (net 2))
 (segment (start 127.54 136.71) (end 127.54 134.125) (width 0.2) (layer "B.Cu") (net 2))
 (segment (start 125.25 137.25) (end 127 137.25) (width 0.2) (layer "B.Cu") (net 2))
 (segment (start 112.301 136.198) (end 112.5 135.999) (width 0.2) (layer "B.Cu") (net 2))
 (segment (start 93.9013 136.198) (end 100.75 136.198) (width 0.2) (layer "B.Cu") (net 2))
 (segment (start 82.25 100.25) (end 82.25 124.5467) (width 0.2) (layer "B.Cu") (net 2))
 (segment (start 82.519997 142.519997) (end 125.675002 142.519997) (width 0.2) (layer "B.Cu") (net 6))
 (segment (start 86.285 90.000003) (end 80.850997 90.000003) (width 0.2) (layer "B.Cu") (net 6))
 (segment (start 80.601 90.25) (end 80.601 140.601) (width 0.2) (layer "B.Cu") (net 6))
 (segment (start 80.601 140.601) (end 82.519997 142.519997) (width 0.2) (layer "B.Cu") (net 6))
 (segment (start 80.850997 90.000003) (end 80.601 90.25) (width 0.2) (layer "B.Cu") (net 6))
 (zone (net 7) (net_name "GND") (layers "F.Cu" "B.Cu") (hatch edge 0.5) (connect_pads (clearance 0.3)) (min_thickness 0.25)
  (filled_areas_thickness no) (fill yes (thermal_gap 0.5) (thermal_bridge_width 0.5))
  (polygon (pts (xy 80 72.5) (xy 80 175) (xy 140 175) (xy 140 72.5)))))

